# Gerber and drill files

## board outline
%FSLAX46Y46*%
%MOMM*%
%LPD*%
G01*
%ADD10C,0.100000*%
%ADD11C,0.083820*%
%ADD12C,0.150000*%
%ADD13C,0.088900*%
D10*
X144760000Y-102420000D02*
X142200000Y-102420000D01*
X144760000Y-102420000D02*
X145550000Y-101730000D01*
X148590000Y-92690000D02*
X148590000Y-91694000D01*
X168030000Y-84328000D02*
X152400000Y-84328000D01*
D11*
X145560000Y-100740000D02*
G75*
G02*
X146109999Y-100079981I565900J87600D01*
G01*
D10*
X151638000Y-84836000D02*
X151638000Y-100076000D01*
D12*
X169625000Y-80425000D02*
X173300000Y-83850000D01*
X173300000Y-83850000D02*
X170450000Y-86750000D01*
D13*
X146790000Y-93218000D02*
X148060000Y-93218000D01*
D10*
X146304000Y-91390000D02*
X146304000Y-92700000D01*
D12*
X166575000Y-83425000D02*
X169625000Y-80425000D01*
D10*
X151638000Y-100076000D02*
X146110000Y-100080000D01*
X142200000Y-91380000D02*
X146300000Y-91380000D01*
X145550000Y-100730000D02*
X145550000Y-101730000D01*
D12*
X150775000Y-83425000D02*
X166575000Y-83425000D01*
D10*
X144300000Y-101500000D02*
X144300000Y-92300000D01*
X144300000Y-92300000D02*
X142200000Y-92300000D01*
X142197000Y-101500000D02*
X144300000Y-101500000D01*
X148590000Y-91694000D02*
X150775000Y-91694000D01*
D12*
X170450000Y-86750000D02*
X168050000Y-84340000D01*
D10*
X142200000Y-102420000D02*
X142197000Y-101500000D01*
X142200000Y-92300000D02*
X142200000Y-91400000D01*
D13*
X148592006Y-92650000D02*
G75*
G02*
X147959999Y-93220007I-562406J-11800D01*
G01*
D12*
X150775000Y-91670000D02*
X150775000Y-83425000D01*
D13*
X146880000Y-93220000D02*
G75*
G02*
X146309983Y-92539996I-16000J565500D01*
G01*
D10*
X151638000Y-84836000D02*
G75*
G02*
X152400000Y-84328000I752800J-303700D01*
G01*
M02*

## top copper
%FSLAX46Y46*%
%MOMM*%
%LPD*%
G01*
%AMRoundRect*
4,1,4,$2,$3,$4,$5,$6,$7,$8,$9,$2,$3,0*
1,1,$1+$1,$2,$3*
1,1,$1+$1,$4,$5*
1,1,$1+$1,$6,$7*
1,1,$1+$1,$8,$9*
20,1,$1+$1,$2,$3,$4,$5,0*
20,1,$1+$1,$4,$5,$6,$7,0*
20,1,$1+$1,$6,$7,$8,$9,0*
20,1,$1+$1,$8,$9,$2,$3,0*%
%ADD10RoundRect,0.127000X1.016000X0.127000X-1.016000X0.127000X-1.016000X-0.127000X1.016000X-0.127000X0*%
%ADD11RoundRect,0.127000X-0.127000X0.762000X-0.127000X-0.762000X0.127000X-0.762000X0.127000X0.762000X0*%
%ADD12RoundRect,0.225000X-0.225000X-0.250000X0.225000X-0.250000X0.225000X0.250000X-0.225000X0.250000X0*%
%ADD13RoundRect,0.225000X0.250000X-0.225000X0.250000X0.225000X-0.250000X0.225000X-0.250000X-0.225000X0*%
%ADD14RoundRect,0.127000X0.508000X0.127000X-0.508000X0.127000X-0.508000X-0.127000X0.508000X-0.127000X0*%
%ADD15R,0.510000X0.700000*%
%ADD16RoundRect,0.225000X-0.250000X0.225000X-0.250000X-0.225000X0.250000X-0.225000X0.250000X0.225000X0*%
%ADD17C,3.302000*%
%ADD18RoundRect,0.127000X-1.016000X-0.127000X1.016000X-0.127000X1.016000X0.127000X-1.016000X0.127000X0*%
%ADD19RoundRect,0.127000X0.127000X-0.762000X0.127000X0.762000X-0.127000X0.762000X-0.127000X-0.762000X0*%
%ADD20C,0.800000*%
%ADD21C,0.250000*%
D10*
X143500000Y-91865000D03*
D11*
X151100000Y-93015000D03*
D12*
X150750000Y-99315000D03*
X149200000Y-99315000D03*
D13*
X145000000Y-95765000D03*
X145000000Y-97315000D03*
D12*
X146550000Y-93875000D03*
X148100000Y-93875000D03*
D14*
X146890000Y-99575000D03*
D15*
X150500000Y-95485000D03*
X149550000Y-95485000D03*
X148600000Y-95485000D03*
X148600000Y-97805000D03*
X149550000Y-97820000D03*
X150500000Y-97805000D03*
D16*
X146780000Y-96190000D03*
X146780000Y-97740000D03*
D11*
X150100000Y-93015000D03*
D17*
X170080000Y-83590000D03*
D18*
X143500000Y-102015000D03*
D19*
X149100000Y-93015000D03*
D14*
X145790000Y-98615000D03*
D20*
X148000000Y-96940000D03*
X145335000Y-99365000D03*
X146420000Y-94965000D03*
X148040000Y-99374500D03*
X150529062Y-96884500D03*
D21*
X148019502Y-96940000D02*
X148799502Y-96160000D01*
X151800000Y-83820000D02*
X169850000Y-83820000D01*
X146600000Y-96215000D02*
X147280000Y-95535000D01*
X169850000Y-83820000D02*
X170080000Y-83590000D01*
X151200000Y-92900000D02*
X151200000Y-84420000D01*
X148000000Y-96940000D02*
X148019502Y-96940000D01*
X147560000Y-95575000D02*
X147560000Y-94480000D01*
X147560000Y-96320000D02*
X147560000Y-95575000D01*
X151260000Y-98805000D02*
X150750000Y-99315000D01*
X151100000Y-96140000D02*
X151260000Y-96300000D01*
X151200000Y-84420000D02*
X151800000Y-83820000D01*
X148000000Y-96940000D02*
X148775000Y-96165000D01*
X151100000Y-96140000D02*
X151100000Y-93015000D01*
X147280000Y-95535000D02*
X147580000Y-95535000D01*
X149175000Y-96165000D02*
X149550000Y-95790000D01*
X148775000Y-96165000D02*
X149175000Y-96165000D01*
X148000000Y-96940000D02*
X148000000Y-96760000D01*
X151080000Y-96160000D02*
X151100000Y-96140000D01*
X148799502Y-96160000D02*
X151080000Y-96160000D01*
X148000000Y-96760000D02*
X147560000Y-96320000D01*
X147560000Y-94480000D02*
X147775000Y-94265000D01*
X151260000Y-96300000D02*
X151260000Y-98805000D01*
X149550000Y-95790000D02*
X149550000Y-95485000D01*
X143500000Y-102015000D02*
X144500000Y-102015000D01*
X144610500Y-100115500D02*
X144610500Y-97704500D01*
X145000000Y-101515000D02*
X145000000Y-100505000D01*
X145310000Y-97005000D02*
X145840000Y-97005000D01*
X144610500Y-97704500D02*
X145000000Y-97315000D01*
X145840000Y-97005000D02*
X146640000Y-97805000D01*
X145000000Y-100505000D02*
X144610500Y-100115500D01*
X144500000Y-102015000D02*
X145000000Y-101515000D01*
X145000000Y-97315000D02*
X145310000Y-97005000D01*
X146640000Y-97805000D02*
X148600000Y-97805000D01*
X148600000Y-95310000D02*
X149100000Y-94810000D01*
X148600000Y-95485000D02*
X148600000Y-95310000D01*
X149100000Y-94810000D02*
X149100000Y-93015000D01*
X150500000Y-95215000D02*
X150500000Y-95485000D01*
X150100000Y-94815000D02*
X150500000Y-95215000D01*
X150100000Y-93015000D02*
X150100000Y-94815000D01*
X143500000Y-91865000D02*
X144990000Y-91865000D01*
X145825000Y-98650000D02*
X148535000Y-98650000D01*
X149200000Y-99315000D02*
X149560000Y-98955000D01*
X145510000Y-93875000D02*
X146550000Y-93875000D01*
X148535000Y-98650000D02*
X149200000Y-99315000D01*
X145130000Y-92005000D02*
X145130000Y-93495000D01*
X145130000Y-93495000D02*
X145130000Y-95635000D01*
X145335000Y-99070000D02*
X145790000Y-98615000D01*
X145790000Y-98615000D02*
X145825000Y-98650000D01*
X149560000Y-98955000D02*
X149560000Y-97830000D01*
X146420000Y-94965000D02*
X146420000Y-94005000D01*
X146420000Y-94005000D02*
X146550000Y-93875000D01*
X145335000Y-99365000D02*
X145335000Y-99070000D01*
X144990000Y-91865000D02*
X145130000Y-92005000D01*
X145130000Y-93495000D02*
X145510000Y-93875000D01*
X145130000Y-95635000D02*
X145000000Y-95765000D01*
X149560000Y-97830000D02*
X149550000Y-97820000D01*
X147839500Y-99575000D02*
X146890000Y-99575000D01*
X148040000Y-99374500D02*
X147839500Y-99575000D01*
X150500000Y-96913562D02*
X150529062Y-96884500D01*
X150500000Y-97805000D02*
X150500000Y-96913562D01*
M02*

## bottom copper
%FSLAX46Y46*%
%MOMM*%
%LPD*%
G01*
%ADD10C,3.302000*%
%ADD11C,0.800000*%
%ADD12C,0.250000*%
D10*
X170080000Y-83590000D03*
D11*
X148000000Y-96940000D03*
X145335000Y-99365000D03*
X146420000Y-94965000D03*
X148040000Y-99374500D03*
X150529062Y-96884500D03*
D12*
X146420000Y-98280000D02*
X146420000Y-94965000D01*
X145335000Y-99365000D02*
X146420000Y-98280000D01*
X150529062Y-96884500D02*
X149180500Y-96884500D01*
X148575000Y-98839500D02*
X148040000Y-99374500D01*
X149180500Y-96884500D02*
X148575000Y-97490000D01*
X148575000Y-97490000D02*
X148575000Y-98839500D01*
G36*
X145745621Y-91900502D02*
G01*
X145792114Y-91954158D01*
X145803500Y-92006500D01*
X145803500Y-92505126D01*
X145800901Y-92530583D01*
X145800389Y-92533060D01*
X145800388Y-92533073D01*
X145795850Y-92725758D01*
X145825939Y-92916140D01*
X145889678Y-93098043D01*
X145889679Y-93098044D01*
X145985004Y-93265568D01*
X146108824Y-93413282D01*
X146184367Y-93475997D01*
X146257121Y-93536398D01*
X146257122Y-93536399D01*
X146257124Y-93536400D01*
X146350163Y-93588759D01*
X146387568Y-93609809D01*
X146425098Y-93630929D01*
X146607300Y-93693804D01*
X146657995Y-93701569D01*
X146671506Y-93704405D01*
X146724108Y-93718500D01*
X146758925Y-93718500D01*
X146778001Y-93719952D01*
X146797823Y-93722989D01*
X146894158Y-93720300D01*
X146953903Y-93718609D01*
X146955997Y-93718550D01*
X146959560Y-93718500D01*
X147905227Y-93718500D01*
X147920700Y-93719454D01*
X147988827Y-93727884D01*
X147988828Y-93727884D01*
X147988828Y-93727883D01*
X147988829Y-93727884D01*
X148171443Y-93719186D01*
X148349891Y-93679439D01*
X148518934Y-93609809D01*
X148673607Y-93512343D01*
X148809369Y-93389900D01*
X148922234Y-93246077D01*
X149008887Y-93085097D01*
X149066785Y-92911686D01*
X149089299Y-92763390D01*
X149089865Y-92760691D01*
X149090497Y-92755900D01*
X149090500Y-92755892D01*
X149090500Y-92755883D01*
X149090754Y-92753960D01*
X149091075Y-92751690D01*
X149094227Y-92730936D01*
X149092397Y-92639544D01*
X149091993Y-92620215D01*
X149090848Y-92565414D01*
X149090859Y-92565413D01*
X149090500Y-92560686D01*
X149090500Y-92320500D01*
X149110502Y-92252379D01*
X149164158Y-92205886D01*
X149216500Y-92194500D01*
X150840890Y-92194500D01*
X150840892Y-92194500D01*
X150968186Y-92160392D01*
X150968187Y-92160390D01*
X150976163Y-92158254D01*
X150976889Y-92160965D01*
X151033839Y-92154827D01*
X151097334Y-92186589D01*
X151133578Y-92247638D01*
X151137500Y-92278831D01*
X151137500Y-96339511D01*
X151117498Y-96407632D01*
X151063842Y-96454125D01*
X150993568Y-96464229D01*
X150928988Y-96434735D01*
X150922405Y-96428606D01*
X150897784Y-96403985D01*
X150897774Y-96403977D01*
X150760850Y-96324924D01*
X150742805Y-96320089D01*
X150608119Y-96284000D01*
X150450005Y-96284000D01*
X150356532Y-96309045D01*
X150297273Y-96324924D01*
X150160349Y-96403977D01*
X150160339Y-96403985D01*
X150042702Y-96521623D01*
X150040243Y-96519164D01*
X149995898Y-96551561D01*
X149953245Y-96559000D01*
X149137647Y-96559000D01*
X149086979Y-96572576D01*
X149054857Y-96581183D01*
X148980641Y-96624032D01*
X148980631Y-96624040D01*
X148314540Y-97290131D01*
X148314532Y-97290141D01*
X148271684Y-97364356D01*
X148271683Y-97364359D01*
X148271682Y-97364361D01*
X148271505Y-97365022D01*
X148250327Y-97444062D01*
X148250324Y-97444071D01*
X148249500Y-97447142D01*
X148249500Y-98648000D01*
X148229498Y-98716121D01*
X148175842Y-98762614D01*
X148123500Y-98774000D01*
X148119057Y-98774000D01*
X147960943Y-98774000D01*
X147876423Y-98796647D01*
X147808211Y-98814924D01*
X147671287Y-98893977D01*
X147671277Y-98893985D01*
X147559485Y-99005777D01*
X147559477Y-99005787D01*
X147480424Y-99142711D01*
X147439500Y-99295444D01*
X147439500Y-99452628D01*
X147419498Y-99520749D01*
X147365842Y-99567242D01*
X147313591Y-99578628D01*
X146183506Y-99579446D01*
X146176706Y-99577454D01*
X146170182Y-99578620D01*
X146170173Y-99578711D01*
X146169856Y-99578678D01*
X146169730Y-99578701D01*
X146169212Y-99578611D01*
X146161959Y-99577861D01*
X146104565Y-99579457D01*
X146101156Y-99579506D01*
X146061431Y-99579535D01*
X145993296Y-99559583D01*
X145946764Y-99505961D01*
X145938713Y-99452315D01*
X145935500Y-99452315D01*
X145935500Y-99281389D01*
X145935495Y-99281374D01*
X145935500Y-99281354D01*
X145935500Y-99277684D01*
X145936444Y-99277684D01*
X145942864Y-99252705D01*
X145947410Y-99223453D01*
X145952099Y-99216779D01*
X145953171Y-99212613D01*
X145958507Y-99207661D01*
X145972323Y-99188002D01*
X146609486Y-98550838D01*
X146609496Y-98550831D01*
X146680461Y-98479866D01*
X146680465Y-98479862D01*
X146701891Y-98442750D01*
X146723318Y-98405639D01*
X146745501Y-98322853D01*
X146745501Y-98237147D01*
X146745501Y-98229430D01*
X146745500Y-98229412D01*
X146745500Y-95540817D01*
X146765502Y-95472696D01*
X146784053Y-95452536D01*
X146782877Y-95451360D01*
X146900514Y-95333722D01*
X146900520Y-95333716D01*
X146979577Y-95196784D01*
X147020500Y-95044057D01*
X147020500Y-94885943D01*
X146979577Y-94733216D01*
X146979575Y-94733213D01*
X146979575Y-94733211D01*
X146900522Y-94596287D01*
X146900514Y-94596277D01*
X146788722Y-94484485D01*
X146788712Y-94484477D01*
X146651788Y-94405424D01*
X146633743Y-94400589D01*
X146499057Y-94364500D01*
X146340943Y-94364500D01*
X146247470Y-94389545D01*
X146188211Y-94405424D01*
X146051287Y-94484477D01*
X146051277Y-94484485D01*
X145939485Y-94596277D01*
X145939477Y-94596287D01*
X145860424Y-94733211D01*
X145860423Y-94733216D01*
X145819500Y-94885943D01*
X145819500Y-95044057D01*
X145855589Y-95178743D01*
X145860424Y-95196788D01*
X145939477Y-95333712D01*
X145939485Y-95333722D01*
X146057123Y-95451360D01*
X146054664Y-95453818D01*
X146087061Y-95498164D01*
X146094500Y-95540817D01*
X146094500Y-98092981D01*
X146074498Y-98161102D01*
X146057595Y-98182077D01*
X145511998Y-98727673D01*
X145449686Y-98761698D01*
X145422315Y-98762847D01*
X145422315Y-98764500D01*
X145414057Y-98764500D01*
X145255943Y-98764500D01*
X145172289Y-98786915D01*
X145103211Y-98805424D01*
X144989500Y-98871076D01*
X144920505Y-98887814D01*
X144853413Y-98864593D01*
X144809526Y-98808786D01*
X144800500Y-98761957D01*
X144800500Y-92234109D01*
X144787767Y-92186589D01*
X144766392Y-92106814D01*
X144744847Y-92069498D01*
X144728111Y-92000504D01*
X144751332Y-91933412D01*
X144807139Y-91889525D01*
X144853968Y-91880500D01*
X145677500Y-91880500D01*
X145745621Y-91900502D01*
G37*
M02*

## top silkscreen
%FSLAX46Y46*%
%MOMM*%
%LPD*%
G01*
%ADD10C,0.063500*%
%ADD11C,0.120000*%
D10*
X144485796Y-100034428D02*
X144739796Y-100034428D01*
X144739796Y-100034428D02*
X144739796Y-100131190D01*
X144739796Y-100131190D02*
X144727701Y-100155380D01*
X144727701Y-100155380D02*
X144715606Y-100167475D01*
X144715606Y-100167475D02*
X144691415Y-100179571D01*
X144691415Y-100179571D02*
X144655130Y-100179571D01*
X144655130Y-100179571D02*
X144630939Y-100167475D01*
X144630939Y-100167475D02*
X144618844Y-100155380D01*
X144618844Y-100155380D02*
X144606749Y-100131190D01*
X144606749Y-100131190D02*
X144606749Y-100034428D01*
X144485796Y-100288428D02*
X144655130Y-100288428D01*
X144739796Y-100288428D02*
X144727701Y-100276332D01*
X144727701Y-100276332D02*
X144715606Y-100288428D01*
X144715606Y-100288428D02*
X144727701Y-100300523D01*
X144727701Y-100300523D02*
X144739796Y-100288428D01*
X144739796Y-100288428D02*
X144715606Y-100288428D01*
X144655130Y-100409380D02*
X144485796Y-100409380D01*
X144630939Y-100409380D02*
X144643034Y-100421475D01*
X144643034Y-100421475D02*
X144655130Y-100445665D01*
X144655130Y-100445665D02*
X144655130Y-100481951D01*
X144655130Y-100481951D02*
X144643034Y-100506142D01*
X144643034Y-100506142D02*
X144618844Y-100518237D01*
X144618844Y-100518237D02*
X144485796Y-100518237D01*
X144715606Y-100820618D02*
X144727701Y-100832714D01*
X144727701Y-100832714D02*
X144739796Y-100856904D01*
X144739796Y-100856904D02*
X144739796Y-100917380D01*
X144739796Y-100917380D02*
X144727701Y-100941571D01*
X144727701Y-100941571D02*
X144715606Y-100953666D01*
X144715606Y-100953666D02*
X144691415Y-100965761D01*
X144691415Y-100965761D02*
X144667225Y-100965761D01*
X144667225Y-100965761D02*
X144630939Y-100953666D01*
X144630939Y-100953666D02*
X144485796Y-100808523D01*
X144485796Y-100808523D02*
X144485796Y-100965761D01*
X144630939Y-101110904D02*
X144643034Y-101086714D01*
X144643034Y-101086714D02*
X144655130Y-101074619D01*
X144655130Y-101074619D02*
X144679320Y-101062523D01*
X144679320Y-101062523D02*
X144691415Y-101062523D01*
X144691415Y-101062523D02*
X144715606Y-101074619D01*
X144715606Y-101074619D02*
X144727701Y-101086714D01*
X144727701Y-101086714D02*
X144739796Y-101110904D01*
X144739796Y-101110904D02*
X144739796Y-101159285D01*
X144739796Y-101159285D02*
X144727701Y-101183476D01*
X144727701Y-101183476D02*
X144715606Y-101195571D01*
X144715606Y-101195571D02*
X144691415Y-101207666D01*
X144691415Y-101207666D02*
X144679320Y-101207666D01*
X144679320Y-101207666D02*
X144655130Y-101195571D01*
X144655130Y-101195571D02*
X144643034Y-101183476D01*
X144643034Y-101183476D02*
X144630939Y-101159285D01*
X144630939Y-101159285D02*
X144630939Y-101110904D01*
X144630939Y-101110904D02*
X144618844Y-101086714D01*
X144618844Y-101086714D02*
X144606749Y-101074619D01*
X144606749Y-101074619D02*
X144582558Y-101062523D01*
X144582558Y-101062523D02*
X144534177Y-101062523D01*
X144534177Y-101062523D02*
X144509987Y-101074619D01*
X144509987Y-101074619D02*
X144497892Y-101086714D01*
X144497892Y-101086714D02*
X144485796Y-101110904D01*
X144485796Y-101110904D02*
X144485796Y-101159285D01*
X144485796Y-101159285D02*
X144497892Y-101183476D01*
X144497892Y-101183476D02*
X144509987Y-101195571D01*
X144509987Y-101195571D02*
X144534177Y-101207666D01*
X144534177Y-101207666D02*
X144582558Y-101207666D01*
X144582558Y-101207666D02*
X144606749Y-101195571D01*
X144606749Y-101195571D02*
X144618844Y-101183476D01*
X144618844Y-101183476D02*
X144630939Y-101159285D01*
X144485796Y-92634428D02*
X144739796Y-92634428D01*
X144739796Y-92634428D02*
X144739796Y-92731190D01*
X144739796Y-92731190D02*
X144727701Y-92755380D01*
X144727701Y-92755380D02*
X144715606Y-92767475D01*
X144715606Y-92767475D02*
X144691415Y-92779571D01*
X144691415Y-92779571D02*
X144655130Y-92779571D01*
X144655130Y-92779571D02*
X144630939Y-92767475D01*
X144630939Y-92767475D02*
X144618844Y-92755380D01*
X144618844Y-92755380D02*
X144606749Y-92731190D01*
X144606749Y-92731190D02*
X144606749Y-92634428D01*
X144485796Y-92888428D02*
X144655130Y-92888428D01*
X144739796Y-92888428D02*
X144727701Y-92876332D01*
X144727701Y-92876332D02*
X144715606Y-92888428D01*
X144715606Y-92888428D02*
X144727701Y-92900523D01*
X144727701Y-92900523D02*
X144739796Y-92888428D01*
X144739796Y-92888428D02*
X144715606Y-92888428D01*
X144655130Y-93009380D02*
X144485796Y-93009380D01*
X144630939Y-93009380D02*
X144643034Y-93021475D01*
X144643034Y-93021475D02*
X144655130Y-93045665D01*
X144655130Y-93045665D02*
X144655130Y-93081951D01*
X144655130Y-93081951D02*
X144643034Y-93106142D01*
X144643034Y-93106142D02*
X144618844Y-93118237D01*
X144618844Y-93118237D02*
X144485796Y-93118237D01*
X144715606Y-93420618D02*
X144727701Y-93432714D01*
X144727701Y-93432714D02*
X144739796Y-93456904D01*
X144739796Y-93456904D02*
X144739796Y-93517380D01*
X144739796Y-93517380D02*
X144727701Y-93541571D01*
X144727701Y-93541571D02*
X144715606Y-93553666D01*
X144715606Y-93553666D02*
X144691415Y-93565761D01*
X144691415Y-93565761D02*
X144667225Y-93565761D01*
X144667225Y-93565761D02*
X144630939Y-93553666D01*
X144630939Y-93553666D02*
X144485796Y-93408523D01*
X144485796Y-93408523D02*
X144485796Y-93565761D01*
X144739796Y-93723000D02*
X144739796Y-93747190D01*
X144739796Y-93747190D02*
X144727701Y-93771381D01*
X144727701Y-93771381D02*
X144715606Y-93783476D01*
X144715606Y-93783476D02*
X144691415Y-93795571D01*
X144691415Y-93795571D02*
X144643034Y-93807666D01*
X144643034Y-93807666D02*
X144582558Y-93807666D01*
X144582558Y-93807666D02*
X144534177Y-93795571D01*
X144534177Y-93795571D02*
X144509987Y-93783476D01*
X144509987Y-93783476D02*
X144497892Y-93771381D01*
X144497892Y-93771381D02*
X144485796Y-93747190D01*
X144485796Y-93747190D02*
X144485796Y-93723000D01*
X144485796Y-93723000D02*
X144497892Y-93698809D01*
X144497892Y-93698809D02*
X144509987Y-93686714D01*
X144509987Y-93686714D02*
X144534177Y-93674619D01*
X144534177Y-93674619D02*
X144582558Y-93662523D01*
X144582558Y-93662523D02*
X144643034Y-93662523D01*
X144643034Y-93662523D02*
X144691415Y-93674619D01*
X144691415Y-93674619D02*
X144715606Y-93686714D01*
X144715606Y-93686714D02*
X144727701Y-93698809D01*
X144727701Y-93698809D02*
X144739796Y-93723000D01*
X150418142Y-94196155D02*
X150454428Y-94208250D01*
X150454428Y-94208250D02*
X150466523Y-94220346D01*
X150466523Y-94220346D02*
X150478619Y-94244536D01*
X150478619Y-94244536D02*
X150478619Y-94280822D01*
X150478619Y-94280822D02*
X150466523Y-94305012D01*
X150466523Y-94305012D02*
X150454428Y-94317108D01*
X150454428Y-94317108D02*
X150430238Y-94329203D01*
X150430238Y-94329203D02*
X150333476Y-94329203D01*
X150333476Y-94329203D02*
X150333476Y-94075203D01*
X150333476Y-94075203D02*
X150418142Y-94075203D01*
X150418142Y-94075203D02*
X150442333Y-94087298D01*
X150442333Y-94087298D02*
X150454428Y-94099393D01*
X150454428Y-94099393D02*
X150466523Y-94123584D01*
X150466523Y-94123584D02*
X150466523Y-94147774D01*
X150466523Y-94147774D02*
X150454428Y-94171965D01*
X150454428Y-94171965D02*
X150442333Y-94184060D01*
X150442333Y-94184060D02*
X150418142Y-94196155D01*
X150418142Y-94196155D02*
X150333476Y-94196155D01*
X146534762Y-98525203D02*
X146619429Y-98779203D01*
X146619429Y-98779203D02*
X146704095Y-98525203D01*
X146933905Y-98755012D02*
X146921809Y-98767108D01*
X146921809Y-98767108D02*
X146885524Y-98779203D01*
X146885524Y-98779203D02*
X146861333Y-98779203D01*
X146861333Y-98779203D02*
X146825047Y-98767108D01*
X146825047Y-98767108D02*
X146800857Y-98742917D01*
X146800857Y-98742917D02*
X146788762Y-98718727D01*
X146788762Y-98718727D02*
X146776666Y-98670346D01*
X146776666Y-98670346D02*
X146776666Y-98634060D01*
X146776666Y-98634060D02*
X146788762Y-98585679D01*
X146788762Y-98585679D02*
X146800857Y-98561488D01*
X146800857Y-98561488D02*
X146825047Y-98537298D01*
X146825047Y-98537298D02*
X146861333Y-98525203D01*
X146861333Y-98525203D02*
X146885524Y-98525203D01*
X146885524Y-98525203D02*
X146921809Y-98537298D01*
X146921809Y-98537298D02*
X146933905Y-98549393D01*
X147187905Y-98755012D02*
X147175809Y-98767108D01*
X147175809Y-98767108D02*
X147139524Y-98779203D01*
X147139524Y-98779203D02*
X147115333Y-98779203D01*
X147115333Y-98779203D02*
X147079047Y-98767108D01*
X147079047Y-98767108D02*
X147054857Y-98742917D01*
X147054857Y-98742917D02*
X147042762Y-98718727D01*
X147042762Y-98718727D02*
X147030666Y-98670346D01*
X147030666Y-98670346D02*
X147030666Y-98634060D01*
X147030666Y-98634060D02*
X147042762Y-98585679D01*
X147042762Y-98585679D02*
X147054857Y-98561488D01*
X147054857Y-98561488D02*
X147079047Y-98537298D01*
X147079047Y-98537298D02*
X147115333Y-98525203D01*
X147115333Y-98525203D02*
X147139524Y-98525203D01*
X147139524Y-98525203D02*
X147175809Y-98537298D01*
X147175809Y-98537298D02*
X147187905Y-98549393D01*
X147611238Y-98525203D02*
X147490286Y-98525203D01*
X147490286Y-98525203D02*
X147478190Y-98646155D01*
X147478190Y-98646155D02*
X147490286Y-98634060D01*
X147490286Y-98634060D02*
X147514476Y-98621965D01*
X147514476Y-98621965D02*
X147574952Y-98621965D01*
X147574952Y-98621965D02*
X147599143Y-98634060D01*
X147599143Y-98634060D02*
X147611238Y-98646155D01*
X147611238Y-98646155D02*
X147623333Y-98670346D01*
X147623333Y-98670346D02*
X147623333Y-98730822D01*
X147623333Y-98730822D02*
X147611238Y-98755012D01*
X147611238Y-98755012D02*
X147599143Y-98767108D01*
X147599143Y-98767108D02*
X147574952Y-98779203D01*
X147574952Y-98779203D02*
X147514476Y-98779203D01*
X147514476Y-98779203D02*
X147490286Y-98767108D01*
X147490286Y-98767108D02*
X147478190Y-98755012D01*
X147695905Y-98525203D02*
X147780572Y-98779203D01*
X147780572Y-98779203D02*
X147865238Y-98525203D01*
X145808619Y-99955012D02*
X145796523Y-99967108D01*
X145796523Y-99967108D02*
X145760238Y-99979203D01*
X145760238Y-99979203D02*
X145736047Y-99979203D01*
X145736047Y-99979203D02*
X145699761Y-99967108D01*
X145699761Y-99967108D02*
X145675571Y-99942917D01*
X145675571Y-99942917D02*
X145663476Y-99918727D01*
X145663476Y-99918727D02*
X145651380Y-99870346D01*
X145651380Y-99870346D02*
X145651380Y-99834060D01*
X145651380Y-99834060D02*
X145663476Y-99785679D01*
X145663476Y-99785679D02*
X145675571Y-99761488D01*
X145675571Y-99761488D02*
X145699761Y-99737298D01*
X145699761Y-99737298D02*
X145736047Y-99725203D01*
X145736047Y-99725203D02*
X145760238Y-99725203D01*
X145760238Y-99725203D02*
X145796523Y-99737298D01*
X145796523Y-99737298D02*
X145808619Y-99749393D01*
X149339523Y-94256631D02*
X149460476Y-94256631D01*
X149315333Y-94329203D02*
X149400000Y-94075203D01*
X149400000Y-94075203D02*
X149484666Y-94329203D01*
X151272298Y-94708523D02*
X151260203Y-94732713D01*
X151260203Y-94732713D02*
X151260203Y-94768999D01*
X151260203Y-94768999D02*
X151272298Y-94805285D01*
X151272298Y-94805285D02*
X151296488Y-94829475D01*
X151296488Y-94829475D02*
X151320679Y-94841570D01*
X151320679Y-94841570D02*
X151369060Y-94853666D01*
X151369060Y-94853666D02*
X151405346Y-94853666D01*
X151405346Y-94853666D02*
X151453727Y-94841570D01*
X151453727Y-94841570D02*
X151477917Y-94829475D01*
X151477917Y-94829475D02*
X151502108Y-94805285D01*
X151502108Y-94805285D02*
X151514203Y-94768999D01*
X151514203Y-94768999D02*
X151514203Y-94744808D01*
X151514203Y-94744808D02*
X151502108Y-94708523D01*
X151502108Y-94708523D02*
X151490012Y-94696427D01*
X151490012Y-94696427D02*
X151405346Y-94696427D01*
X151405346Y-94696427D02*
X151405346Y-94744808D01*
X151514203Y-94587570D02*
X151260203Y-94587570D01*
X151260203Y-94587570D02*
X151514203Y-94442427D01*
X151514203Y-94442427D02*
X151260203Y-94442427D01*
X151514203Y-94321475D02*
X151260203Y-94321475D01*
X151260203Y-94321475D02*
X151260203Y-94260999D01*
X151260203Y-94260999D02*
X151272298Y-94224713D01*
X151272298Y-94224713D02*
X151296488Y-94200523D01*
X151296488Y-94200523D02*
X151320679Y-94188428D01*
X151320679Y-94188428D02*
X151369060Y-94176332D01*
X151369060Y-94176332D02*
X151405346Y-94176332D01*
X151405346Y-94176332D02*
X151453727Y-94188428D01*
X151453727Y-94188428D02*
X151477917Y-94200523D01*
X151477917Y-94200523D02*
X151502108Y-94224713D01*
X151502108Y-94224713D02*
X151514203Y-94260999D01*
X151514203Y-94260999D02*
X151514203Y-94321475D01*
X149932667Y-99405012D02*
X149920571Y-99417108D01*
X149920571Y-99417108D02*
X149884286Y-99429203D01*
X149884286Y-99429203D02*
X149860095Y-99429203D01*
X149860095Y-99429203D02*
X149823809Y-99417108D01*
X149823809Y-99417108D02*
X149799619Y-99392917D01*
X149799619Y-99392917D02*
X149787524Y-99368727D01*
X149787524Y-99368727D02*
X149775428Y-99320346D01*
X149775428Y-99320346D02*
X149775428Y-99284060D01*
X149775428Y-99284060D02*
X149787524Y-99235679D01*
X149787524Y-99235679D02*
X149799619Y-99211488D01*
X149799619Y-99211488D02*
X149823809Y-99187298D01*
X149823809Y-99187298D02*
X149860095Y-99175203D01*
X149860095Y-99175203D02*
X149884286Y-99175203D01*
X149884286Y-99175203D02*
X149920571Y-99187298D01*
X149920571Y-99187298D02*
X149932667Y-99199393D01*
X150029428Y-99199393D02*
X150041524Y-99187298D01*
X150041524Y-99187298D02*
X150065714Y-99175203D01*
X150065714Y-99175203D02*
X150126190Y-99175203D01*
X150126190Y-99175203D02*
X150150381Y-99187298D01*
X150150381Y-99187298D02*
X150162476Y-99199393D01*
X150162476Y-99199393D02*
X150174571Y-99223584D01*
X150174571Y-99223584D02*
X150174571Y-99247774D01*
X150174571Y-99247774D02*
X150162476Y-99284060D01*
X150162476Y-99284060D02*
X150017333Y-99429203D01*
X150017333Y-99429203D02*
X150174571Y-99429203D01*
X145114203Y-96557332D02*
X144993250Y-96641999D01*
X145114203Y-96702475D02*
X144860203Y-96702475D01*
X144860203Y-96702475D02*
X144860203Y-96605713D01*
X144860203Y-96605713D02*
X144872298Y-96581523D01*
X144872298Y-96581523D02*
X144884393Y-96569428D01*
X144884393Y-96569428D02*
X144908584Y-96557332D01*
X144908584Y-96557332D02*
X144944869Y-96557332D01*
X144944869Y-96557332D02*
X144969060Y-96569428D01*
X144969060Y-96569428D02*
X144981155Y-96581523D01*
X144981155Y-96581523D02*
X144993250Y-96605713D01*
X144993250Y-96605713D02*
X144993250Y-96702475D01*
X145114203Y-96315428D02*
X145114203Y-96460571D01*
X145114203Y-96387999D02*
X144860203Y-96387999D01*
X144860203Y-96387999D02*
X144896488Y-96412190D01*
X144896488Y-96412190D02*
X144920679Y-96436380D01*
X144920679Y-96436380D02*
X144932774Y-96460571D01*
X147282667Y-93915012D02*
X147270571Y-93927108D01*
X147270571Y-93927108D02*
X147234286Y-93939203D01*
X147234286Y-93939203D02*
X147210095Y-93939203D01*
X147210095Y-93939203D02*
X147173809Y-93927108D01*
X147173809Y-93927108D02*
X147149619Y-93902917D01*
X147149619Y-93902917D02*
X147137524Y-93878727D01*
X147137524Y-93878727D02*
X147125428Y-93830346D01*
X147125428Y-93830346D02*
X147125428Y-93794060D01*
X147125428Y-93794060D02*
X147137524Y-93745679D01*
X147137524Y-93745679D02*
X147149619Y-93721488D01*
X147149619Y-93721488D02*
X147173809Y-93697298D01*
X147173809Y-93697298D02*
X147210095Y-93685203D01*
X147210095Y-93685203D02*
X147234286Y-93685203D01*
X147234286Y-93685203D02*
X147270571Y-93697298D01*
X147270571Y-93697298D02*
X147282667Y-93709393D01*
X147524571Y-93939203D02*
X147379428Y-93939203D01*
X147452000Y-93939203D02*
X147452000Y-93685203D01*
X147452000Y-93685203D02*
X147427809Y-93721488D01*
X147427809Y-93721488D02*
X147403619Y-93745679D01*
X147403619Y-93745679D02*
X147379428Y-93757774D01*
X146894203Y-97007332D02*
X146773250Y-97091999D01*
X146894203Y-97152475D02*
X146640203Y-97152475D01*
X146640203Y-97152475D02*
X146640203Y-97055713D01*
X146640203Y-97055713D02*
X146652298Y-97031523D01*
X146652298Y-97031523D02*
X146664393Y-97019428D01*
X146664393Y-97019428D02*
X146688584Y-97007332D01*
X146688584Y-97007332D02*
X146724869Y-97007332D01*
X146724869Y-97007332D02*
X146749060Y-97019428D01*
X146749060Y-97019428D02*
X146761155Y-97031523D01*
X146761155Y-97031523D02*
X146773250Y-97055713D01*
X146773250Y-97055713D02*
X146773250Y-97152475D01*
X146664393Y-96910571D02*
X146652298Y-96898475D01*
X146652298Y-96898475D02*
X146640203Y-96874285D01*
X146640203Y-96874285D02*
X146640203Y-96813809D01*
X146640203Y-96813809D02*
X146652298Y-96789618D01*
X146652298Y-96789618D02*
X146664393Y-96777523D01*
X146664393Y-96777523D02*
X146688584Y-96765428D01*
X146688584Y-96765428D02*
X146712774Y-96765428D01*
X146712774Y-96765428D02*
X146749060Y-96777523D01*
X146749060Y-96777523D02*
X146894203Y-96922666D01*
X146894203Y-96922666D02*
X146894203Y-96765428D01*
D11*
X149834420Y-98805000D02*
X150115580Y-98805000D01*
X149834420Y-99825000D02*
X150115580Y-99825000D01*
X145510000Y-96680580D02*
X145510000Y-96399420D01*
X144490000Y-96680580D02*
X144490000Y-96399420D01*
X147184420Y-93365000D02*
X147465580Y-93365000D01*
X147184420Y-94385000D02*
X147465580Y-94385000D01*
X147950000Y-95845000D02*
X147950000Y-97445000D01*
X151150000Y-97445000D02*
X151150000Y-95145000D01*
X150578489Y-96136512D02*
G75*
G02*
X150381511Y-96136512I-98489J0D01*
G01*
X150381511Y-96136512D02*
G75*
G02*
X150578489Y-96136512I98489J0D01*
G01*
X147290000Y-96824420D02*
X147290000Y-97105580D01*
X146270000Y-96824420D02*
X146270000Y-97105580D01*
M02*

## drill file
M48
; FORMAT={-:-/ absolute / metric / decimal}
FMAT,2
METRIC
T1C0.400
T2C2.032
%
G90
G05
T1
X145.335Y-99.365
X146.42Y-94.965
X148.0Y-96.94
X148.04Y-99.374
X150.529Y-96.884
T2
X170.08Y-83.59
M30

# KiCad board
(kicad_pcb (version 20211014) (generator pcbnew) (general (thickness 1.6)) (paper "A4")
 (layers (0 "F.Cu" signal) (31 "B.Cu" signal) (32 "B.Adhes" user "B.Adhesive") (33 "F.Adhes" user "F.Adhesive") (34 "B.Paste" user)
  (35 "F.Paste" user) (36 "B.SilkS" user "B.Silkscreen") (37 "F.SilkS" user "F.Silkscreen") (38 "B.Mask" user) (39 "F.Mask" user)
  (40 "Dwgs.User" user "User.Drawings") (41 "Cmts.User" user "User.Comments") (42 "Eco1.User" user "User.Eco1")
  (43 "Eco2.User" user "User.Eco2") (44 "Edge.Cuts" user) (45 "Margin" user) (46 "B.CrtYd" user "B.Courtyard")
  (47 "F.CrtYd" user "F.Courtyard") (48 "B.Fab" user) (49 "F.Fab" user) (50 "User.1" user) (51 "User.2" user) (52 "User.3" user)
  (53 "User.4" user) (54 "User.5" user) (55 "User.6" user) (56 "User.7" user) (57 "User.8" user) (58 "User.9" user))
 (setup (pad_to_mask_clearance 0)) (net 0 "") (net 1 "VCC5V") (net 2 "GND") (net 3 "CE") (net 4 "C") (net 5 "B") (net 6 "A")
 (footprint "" (layer "F.Cu") (at 143.5 91.865 180)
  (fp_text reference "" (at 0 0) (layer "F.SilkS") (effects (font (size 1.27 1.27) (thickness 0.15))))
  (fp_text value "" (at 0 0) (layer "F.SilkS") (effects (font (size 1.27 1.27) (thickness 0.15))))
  (pad "1" smd roundrect (at 0 0 180) (size 2.286 0.508) (layers "F.Cu" "F.Paste" "F.Mask") (roundrect_rratio 0.25) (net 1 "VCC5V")))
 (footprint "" (layer "F.Cu") (at 151.1 93.015 90)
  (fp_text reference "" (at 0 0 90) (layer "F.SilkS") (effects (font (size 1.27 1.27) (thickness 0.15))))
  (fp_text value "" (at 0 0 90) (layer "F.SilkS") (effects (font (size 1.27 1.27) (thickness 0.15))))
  (pad "9" smd roundrect (at 0 0 270) (size 1.778 0.508) (layers "F.Cu" "F.Paste" "F.Mask") (roundrect_rratio 0.25) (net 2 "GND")))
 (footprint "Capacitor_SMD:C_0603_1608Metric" (layer "F.Cu") (at 149.975 99.315)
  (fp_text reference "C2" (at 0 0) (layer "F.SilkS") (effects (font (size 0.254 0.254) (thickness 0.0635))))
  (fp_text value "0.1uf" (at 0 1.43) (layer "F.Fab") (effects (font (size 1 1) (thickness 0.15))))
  (fp_line (start -0.14058 -0.51) (end 0.14058 -0.51) (layer "F.SilkS") (width 0.12))
  (fp_line (start -0.14058 0.51) (end 0.14058 0.51) (layer "F.SilkS") (width 0.12))
  (pad "7" smd roundrect (at 0.775 0) (size 0.9 0.95) (layers "F.Cu" "F.Paste" "F.Mask") (roundrect_rratio 0.25) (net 2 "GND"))
  (pad "8" smd roundrect (at -0.775 0) (size 0.9 0.95) (layers "F.Cu" "F.Paste" "F.Mask") (roundrect_rratio 0.25) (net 1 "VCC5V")))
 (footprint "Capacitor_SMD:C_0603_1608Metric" (layer "F.Cu") (at 145 96.54 90)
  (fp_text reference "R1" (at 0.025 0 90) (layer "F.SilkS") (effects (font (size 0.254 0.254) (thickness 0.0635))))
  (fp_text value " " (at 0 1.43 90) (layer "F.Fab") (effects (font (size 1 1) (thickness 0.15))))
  (fp_line (start -0.14058 0.51) (end 0.14058 0.51) (layer "F.SilkS") (width 0.12))
  (fp_line (start -0.14058 -0.51) (end 0.14058 -0.51) (layer "F.SilkS") (width 0.12))
  (pad "2" smd roundrect (at 0.775 0 90) (size 0.9 0.95) (layers "F.Cu" "F.Paste" "F.Mask") (roundrect_rratio 0.25) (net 1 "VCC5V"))
  (pad "3" smd roundrect (at -0.775 0 90) (size 0.9 0.95) (layers "F.Cu" "F.Paste" "F.Mask") (roundrect_rratio 0.25) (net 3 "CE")))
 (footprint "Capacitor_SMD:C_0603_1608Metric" (layer "F.Cu") (at 147.325 93.875)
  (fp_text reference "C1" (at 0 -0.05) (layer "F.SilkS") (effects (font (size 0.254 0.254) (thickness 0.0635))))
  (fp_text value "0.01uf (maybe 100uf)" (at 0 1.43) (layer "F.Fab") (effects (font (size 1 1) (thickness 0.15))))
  (fp_line (start -0.14058 -0.51) (end 0.14058 -0.51) (layer "F.SilkS") (width 0.12))
  (fp_line (start -0.14058 0.51) (end 0.14058 0.51) (layer "F.SilkS") (width 0.12))
  (pad "5" smd roundrect (at -0.775 0) (size 0.9 0.95) (layers "F.Cu" "F.Paste" "F.Mask") (roundrect_rratio 0.25) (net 1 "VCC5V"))
  (pad "6" smd roundrect (at 0.775 0) (size 0.9 0.95) (layers "F.Cu" "F.Paste" "F.Mask") (roundrect_rratio 0.25) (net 2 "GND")))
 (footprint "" (layer "F.Cu") (at 146.89 99.575)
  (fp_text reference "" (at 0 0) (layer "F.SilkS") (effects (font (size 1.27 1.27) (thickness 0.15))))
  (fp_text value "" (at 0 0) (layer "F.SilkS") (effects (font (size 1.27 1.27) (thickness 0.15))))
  (pad "B" smd roundrect (at 0 0 180) (size 1.27 0.508) (layers "F.Cu" "F.Paste" "F.Mask") (roundrect_rratio 0.25) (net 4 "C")))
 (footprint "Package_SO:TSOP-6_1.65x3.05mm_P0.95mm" (layer "F.Cu") (at 149.55 96.645 -90)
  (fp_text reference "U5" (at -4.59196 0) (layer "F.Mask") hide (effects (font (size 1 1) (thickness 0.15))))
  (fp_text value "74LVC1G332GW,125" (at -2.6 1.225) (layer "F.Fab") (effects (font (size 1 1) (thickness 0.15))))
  (fp_line (start -0.8 1.6) (end 0.8 1.6) (layer "F.SilkS") (width 0.12))
  (fp_line (start 0.8 -1.6) (end -1.5 -1.6) (layer "F.SilkS") (width 0.12))
  (fp_circle (center -0.508488 -0.93) (end -0.418488 -0.89) (layer "F.SilkS") (width 0.12) (fill none))
  (pad "1" smd rect (at -1.16 -0.95 270) (size 0.7 0.51) (layers "F.Cu" "F.Paste" "F.Mask") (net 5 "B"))
  (pad "2" smd rect (at -1.16 0 270) (size 0.7 0.51) (layers "F.Cu" "F.Paste" "F.Mask") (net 2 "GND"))
  (pad "3" smd rect (at -1.16 0.95 270) (size 0.7 0.51) (layers "F.Cu" "F.Paste" "F.Mask") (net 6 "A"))
  (pad "4" smd rect (at 1.16 0.95 270) (size 0.7 0.51) (layers "F.Cu" "F.Paste" "F.Mask") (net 3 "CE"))
  (pad "5" smd rect (at 1.175 0 270) (size 0.7 0.51) (layers "F.Cu" "F.Paste" "F.Mask") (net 1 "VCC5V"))
  (pad "6" smd rect (at 1.16 -0.95 270) (size 0.7 0.51) (layers "F.Cu" "F.Paste" "F.Mask") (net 4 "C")))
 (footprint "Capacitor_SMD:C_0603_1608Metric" (layer "F.Cu") (at 146.78 96.965 -90)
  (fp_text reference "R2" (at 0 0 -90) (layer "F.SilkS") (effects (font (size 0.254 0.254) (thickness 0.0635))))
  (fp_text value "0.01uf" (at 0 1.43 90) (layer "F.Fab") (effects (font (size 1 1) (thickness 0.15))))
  (fp_line (start -0.14058 -0.51) (end 0.14058 -0.51) (layer "F.SilkS") (width 0.12))
  (fp_line (start -0.14058 0.51) (end 0.14058 0.51) (layer "F.SilkS") (width 0.12))
  (pad "5" smd roundrect (at -0.775 0 270) (size 0.9 0.95) (layers "F.Cu" "F.Paste" "F.Mask") (roundrect_rratio 0.25) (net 2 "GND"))
  (pad "6" smd roundrect (at 0.775 0 270) (size 0.9 0.95) (layers "F.Cu" "F.Paste" "F.Mask") (roundrect_rratio 0.25) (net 3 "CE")))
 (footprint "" (layer "F.Cu") (at 150.1 93.015 90)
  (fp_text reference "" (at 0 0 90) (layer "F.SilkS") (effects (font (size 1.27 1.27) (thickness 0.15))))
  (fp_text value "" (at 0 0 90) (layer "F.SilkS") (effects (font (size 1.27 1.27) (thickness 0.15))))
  (pad "10" smd roundrect (at 0 0 270) (size 1.778 0.508) (layers "F.Cu" "F.Paste" "F.Mask") (roundrect_rratio 0.25) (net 5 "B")))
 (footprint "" (layer "F.Cu") (at 170.08 83.59)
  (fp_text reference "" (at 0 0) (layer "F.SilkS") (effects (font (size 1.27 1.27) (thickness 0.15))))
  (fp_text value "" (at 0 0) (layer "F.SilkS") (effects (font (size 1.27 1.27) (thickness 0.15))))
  (pad "9" thru_hole circle (at 0 0 270) (size 3.302 3.302) (drill 2.032) (layers *.Cu *.Mask) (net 2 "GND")))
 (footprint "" (layer "F.Cu") (at 143.5 102.015)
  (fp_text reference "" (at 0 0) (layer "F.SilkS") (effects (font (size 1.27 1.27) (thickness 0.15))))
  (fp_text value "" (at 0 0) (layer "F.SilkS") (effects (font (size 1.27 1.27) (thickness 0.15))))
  (pad "4" smd roundrect (at 0 0) (size 2.286 0.508) (layers "F.Cu" "F.Paste" "F.Mask") (roundrect_rratio 0.25) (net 3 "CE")))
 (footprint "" (layer "F.Cu") (at 149.1 93.015 -90)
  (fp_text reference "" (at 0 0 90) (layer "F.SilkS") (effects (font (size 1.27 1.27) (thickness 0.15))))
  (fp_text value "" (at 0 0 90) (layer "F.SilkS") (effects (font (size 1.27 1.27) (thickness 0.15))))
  (pad "11" smd roundrect (at 0 0 90) (size 1.778 0.508) (layers "F.Cu" "F.Paste" "F.Mask") (roundrect_rratio 0.25) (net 6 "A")))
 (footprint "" (layer "F.Cu") (at 145.79 98.615 -90)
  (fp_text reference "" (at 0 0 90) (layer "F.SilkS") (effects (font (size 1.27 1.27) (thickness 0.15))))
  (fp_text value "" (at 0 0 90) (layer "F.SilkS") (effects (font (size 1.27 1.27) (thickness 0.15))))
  (pad "B" smd roundrect (at 0 0 180) (size 1.27 0.508) (layers "F.Cu" "F.Paste" "F.Mask") (roundrect_rratio 0.25) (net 1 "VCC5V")))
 (gr_line (start 144.76 102.42) (end 142.2 102.42) (layer "Edge.Cuts") (width 0.1))
 (gr_line (start 144.76 102.42) (end 145.55 101.73) (layer "Edge.Cuts") (width 0.1))
 (gr_line (start 148.59 92.69) (end 148.59 91.694) (layer "Edge.Cuts") (width 0.1))
 (gr_line (start 168.03 84.328) (end 152.4 84.328) (layer "Edge.Cuts") (width 0.1))
 (gr_arc (start 145.56 100.74) (mid 145.684497 100.28762) (end 146.11 100.08) (layer "Edge.Cuts") (width 0.08382))
 (gr_line (start 151.638 84.836) (end 151.638 100.076) (layer "Edge.Cuts") (width 0.1))
 (gr_line (start 169.625 80.425) (end 173.3 83.85) (layer "Edge.Cuts") (width 0.15))
 (gr_line (start 173.3 83.85) (end 170.45 86.75) (layer "Edge.Cuts") (width 0.15))
 (gr_line (start 146.79 93.218) (end 148.06 93.218) (layer "Edge.Cuts") (width 0.0889))
 (gr_line (start 146.304 91.39) (end 146.304 92.7) (layer "Edge.Cuts") (width 0.1))
 (gr_line (start 166.575 83.425) (end 169.625 80.425) (layer "Edge.Cuts") (width 0.15))
 (gr_line (start 151.638 100.076) (end 146.11 100.08) (layer "Edge.Cuts") (width 0.1))
 (gr_line (start 142.2 91.38) (end 146.3 91.38) (layer "Edge.Cuts") (width 0.1))
 (gr_line (start 145.55 100.73) (end 145.55 101.73) (layer "Edge.Cuts") (width 0.1))
 (gr_line (start 150.775 83.425) (end 166.575 83.425) (layer "Edge.Cuts") (width 0.15))
 (gr_line (start 144.3 101.5) (end 144.3 92.3) (layer "Edge.Cuts") (width 0.1))
 (gr_line (start 144.3 92.3) (end 142.2 92.3) (layer "Edge.Cuts") (width 0.1))
 (gr_line (start 142.197 101.5) (end 144.3 101.5) (layer "Edge.Cuts") (width 0.1))
 (gr_line (start 148.59 91.694) (end 150.775 91.694) (layer "Edge.Cuts") (width 0.1))
 (gr_line (start 170.45 86.75) (end 168.05 84.34) (layer "Edge.Cuts") (width 0.15))
 (gr_line (start 142.2 102.42) (end 142.197 101.5) (layer "Edge.Cuts") (width 0.1))
 (gr_line (start 142.2 92.3) (end 142.2 91.4) (layer "Edge.Cuts") (width 0.1))
 (gr_arc (start 148.592006 92.65) (mid 148.406336 93.079511) (end 147.96 93.22) (layer "Edge.Cuts") (width 0.0889))
 (gr_line (start 150.775 91.67) (end 150.775 83.425) (layer "Edge.Cuts") (width 0.15))
 (gr_arc (start 146.88 93.22) (mid 146.430454 93.017928) (end 146.31 92.54) (layer "Edge.Cuts") (width 0.0889))
 (gr_arc (start 151.638 84.836) (mid 151.940524 84.464286) (end 152.4 84.328) (layer "Edge.Cuts") (width 0.1))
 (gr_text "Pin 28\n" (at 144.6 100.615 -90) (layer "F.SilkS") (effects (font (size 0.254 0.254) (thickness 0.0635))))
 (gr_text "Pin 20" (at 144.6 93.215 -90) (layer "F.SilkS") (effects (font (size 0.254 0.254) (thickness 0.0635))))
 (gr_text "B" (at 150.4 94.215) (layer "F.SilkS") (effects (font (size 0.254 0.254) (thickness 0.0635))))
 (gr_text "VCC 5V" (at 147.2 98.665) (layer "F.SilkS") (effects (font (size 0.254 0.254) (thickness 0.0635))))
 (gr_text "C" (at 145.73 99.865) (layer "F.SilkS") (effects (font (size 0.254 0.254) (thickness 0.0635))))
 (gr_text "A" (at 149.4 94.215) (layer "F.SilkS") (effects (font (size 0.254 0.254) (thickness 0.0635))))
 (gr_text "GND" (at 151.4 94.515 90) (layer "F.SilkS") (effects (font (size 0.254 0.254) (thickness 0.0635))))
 (segment (start 148.019502 96.94) (end 148.799502 96.16) (width 0.25) (layer "F.Cu") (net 2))
 (segment (start 151.8 83.82) (end 169.85 83.82) (width 0.25) (layer "F.Cu") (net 2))
 (segment (start 146.6 96.215) (end 147.28 95.535) (width 0.25) (layer "F.Cu") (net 2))
 (segment (start 169.85 83.82) (end 170.08 83.59) (width 0.25) (layer "F.Cu") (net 2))
 (segment (start 151.2 92.9) (end 151.2 84.42) (width 0.25) (layer "F.Cu") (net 2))
 (segment (start 148 96.94) (end 148.019502 96.94) (width 0.25) (layer "F.Cu") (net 2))
 (segment (start 147.56 95.575) (end 147.56 94.48) (width 0.25) (layer "F.Cu") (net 2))
 (segment (start 147.56 96.32) (end 147.56 95.575) (width 0.25) (layer "F.Cu") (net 2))
 (segment (start 151.26 98.805) (end 150.75 99.315) (width 0.25) (layer "F.Cu") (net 2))
 (segment (start 151.1 96.14) (end 151.26 96.3) (width 0.25) (layer "F.Cu") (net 2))
 (segment (start 151.2 84.42) (end 151.8 83.82) (width 0.25) (layer "F.Cu") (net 2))
 (segment (start 148 96.94) (end 148.775 96.165) (width 0.25) (layer "F.Cu") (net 2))
 (segment (start 151.1 96.14) (end 151.1 93.015) (width 0.25) (layer "F.Cu") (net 2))
 (segment (start 147.28 95.535) (end 147.58 95.535) (width 0.25) (layer "F.Cu") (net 2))
 (segment (start 149.175 96.165) (end 149.55 95.79) (width 0.25) (layer "F.Cu") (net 2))
 (segment (start 148.775 96.165) (end 149.175 96.165) (width 0.25) (layer "F.Cu") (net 2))
 (segment (start 148 96.94) (end 148 96.76) (width 0.25) (layer "F.Cu") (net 2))
 (segment (start 151.08 96.16) (end 151.1 96.14) (width 0.25) (layer "F.Cu") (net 2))
 (segment (start 148.799502 96.16) (end 151.08 96.16) (width 0.25) (layer "F.Cu") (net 2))
 (segment (start 148 96.76) (end 147.56 96.32) (width 0.25) (layer "F.Cu") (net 2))
 (segment (start 147.56 94.48) (end 147.775 94.265) (width 0.25) (layer "F.Cu") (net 2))
 (segment (start 151.26 96.3) (end 151.26 98.805) (width 0.25) (layer "F.Cu") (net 2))
 (segment (start 149.55 95.79) (end 149.55 95.485) (width 0.25) (layer "F.Cu") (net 2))
 (via (at 148 96.94) (size 0.8) (drill 0.4) (layers "F.Cu" "B.Cu") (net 2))
 (segment (start 143.5 102.015) (end 144.5 102.015) (width 0.25) (layer "F.Cu") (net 3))
 (segment (start 144.6105 100.1155) (end 144.6105 97.7045) (width 0.25) (layer "F.Cu") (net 3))
 (segment (start 145 101.515) (end 145 100.505) (width 0.25) (layer "F.Cu") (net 3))
 (segment (start 145.31 97.005) (end 145.84 97.005) (width 0.25) (layer "F.Cu") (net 3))
 (segment (start 144.6105 97.7045) (end 145 97.315) (width 0.25) (layer "F.Cu") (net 3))
 (segment (start 145.84 97.005) (end 146.64 97.805) (width 0.25) (layer "F.Cu") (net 3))
 (segment (start 145 100.505) (end 144.6105 100.1155) (width 0.25) (layer "F.Cu") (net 3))
 (segment (start 144.5 102.015) (end 145 101.515) (width 0.25) (layer "F.Cu") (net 3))
 (segment (start 145 97.315) (end 145.31 97.005) (width 0.25) (layer "F.Cu") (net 3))
 (segment (start 146.64 97.805) (end 148.6 97.805) (width 0.25) (layer "F.Cu") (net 3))
 (segment (start 148.6 95.31) (end 149.1 94.81) (width 0.25) (layer "F.Cu") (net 6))
 (segment (start 148.6 95.485) (end 148.6 95.31) (width 0.25) (layer "F.Cu") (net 6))
 (segment (start 149.1 94.81) (end 149.1 93.015) (width 0.25) (layer "F.Cu") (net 6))
 (segment (start 150.5 95.215) (end 150.5 95.485) (width 0.25) (layer "F.Cu") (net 5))
 (segment (start 150.1 94.815) (end 150.5 95.215) (width 0.25) (layer "F.Cu") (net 5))
 (segment (start 150.1 93.015) (end 150.1 94.815) (width 0.25) (layer "F.Cu") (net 5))
 (segment (start 143.5 91.865) (end 144.99 91.865) (width 0.25) (layer "F.Cu") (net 1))
 (segment (start 145.825 98.65) (end 148.535 98.65) (width 0.25) (layer "F.Cu") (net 1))
 (segment (start 149.2 99.315) (end 149.56 98.955) (width 0.25) (layer "F.Cu") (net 1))
 (segment (start 145.51 93.875) (end 146.55 93.875) (width 0.25) (layer "F.Cu") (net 1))
 (segment (start 148.535 98.65) (end 149.2 99.315) (width 0.25) (layer "F.Cu") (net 1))
 (segment (start 145.13 92.005) (end 145.13 93.495) (width 0.25) (layer "F.Cu") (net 1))
 (segment (start 145.13 93.495) (end 145.13 95.635) (width 0.25) (layer "F.Cu") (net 1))
 (segment (start 145.335 99.07) (end 145.79 98.615) (width 0.25) (layer "F.Cu") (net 1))
 (segment (start 145.79 98.615) (end 145.825 98.65) (width 0.25) (layer "F.Cu") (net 1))
 (segment (start 149.56 98.955) (end 149.56 97.83) (width 0.25) (layer "F.Cu") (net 1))
 (segment (start 146.42 94.965) (end 146.42 94.005) (width 0.25) (layer "F.Cu") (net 1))
 (segment (start 146.42 94.005) (end 146.55 93.875) (width 0.25) (layer "F.Cu") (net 1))
 (segment (start 145.335 99.365) (end 145.335 99.07) (width 0.25) (layer "F.Cu") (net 1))
 (segment (start 144.99 91.865) (end 145.13 92.005) (width 0.25) (layer "F.Cu") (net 1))
 (segment (start 145.13 93.495) (end 145.51 93.875) (width 0.25) (layer "F.Cu") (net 1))
 (segment (start 145.13 95.635) (end 145 95.765) (width 0.25) (layer "F.Cu") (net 1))
 (segment (start 149.56 97.83) (end 149.55 97.82) (width 0.25) (layer "F.Cu") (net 1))
 (via (at 145.335 99.365) (size 0.8) (drill 0.4) (layers "F.Cu" "B.Cu") (free) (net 1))
 (via (at 146.42 94.965) (size 0.8) (drill 0.4) (layers "F.Cu" "B.Cu") (free) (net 1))
 (segment (start 146.42 98.28) (end 146.42 94.965) (width 0.25) (layer "B.Cu") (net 1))
 (segment (start 145.335 99.365) (end 146.42 98.28) (width 0.25) (layer "B.Cu") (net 1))
 (segment (start 147.8395 99.575) (end 146.89 99.575) (width 0.25) (layer "F.Cu") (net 4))
 (segment (start 148.04 99.3745) (end 147.8395 99.575) (width 0.25) (layer "F.Cu") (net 4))
 (segment (start 150.5 96.913562) (end 150.529062 96.8845) (width 0.25) (layer "F.Cu") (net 4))
 (segment (start 150.5 97.805) (end 150.5 96.913562) (width 0.25) (layer "F.Cu") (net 4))
 (via (at 148.04 99.3745) (size 0.8) (drill 0.4) (layers "F.Cu" "B.Cu") (free) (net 4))
 (via (at 150.529062 96.8845) (size 0.8) (drill 0.4) (layers "F.Cu" "B.Cu") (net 4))
 (segment (start 150.529062 96.8845) (end 149.1805 96.8845) (width 0.25) (layer "B.Cu") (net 4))
 (segment (start 148.575 98.8395) (end 148.04 99.3745) (width 0.25) (layer "B.Cu") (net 4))
 (segment (start 149.1805 96.8845) (end 148.575 97.49) (width 0.25) (layer "B.Cu") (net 4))
 (segment (start 148.575 97.49) (end 148.575 98.8395) (width 0.25) (layer "B.Cu") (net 4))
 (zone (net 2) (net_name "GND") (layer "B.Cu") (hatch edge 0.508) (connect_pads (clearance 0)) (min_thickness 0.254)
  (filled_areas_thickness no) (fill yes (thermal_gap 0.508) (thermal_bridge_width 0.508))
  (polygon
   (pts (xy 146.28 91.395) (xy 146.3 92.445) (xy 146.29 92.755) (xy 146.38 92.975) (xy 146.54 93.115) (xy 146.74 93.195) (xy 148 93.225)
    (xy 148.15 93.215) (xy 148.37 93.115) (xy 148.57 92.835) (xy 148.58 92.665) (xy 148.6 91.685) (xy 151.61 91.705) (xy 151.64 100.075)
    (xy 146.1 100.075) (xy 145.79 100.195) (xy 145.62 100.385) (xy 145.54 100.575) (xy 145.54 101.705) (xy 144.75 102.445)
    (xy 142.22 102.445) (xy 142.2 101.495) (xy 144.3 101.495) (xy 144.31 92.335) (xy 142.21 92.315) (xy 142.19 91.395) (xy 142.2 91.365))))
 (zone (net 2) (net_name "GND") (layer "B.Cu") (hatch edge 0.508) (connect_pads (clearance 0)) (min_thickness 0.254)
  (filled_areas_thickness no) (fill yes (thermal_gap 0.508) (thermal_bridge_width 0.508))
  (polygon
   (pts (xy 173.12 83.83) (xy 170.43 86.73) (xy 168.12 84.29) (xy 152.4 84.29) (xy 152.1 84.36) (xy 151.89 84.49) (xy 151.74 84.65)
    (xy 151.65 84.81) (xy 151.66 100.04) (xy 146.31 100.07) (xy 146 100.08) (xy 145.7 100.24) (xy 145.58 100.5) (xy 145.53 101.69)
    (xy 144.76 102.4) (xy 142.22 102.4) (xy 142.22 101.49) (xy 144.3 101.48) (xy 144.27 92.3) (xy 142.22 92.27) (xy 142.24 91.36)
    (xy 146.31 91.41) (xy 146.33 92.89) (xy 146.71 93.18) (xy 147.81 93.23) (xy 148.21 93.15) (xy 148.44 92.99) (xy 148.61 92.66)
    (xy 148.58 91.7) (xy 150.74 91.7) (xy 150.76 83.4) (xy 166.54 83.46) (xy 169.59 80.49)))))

